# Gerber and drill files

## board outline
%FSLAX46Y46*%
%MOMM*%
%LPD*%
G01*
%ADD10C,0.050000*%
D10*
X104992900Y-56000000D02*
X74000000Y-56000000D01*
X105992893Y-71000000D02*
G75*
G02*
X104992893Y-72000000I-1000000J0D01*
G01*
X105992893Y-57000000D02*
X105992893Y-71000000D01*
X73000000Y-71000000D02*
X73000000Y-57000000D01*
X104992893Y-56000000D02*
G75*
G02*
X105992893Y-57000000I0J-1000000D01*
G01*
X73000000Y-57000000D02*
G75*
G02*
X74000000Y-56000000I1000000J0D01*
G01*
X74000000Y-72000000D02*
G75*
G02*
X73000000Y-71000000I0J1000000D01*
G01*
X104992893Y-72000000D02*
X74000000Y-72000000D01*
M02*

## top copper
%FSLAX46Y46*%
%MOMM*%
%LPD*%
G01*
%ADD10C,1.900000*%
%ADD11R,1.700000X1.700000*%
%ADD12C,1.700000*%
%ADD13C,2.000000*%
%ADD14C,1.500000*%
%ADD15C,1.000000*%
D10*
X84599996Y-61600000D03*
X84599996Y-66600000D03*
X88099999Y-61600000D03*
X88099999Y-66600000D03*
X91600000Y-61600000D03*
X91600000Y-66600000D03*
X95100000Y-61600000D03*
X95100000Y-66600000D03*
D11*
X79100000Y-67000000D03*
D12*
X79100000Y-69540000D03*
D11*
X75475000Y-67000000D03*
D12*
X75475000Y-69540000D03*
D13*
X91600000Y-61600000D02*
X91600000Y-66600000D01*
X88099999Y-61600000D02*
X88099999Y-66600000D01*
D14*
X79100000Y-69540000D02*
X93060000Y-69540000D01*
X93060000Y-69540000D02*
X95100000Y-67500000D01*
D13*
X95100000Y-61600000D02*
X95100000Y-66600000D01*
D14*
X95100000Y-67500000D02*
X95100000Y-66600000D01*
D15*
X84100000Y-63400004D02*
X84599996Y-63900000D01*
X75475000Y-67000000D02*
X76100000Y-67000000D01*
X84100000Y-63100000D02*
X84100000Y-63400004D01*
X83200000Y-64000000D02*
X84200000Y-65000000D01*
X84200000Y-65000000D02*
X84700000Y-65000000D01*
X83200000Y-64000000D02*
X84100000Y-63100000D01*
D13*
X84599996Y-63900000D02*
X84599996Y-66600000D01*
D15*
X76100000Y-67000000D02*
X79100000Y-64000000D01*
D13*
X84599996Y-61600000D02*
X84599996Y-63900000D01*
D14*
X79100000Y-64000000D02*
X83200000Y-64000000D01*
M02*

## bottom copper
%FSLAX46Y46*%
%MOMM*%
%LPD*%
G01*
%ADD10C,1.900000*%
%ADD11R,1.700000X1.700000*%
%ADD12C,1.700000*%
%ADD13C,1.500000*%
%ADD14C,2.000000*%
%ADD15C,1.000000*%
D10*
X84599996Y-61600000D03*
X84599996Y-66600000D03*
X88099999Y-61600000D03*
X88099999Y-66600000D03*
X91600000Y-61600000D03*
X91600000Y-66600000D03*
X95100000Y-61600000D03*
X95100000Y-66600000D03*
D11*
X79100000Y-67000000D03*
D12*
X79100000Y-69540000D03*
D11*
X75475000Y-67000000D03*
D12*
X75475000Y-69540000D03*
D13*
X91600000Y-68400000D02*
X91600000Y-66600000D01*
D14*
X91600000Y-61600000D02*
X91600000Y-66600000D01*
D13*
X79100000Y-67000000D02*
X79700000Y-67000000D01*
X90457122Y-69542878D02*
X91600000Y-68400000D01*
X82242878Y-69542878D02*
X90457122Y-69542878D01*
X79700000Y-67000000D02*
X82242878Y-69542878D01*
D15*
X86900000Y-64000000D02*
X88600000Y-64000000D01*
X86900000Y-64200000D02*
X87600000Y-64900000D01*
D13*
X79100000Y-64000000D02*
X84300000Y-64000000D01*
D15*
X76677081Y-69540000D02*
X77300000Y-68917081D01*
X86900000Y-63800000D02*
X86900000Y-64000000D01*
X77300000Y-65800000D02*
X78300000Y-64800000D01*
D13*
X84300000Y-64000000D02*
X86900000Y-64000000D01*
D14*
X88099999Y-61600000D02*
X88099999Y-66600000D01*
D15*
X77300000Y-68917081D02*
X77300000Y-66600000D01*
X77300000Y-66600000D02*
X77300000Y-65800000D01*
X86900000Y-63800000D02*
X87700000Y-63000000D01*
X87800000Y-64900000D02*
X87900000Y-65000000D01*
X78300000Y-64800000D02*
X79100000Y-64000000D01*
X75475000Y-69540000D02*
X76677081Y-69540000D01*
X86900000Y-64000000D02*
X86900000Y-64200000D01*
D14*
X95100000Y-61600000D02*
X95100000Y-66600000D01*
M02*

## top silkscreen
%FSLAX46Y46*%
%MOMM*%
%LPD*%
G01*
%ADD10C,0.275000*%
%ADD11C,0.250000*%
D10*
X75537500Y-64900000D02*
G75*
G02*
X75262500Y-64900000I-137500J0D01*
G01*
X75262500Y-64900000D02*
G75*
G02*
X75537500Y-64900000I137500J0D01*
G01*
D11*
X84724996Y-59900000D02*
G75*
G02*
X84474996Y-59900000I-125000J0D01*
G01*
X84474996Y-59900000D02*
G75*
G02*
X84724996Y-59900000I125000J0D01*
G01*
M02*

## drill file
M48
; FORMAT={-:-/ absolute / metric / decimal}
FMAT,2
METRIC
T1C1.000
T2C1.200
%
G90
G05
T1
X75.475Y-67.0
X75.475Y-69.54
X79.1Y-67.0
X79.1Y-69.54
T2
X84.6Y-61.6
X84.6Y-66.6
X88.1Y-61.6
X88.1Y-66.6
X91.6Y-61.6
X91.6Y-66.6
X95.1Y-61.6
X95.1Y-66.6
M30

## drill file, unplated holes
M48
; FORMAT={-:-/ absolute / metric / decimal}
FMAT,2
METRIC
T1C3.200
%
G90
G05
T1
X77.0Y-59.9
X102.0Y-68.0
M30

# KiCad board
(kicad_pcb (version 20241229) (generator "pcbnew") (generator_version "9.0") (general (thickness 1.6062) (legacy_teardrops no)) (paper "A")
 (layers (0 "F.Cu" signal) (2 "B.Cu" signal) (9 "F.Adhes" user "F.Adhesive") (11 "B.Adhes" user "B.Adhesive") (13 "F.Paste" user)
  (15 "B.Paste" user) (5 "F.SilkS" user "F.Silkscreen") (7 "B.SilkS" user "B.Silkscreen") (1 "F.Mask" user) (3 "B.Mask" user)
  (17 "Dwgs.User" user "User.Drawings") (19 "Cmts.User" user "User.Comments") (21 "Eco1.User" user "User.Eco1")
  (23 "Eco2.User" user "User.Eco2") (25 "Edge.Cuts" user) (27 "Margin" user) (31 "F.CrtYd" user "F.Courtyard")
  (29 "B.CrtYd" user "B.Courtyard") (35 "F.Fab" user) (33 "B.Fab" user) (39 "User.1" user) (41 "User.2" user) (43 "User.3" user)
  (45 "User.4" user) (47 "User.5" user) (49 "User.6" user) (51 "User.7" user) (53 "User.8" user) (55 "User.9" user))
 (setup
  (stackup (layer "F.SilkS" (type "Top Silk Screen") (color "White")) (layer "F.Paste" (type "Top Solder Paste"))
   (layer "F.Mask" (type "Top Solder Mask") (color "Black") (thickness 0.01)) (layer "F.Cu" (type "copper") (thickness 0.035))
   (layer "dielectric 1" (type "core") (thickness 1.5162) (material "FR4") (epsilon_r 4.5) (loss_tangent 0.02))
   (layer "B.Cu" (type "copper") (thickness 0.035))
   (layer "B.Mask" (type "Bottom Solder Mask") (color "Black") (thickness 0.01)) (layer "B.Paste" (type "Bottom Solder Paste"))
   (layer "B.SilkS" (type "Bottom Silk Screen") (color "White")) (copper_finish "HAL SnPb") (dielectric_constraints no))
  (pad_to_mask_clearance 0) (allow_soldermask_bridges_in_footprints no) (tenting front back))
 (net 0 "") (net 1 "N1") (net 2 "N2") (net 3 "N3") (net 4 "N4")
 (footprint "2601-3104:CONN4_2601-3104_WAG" (layer "F.Cu") (at 84.599996 61.6)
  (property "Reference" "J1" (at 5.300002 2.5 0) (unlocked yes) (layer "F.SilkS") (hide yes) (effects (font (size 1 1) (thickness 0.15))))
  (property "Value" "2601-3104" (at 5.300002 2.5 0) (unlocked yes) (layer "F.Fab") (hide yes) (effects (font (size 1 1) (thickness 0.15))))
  (fp_circle (center 0 -1.7) (end 0.2 -1.7) (stroke (width 0.1) (type solid)) (fill yes) (layer "F.SilkS"))
  (pad "1" thru_hole circle (at 0 0) (size 1.9 1.9) (drill 1.2) (layers "*.Cu" "*.Mask") (remove_unused_layers no) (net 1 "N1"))
  (pad "1" thru_hole circle (at 0 5) (size 1.9 1.9) (drill 1.2) (layers "*.Cu" "*.Mask") (remove_unused_layers no) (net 1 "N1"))
  (pad "2" thru_hole circle (at 3.500003 0) (size 1.9 1.9) (drill 1.2) (layers "*.Cu" "*.Mask") (remove_unused_layers no) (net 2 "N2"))
  (pad "2" thru_hole circle (at 3.500003 5) (size 1.9 1.9) (drill 1.2) (layers "*.Cu" "*.Mask") (remove_unused_layers no) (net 2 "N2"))
  (pad "3" thru_hole circle (at 7.000004 0) (size 1.9 1.9) (drill 1.2) (layers "*.Cu" "*.Mask") (remove_unused_layers no) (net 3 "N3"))
  (pad "3" thru_hole circle (at 7.000004 5) (size 1.9 1.9) (drill 1.2) (layers "*.Cu" "*.Mask") (remove_unused_layers no) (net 3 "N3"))
  (pad "4" thru_hole circle (at 10.500004 0) (size 1.9 1.9) (drill 1.2) (layers "*.Cu" "*.Mask") (remove_unused_layers no) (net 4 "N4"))
  (pad "4" thru_hole circle (at 10.500004 5) (size 1.9 1.9) (drill 1.2) (layers "*.Cu" "*.Mask") (remove_unused_layers no) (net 4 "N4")))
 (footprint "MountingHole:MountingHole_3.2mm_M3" (layer "F.Cu") (at 102 68)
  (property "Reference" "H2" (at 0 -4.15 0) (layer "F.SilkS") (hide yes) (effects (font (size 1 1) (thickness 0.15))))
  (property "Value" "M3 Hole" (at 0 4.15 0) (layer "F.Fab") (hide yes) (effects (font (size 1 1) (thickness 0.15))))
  (pad "" np_thru_hole circle (at 0 0) (size 3.2 3.2) (drill 3.2) (layers "*.Cu" "*.Mask")))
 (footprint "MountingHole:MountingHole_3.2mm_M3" (layer "F.Cu") (at 77 59.9)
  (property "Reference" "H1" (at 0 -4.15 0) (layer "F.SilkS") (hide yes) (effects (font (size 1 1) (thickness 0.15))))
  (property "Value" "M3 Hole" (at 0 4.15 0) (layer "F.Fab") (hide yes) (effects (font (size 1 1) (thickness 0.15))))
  (pad "" np_thru_hole circle (at 0 0) (size 3.2 3.2) (drill 3.2) (layers "*.Cu" "*.Mask")))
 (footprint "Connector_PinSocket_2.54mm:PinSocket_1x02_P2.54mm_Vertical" (layer "B.Cu") (at 79.1 67 180)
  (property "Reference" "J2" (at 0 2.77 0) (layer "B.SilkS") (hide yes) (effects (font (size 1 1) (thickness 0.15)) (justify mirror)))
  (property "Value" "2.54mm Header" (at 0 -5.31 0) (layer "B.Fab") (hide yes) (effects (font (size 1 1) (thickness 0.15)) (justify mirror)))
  (pad "1" thru_hole rect (at 0 0 180) (size 1.7 1.7) (drill 1) (layers "*.Cu" "*.Mask") (remove_unused_layers no) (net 3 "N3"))
  (pad "2" thru_hole circle (at 0 -2.54 180) (size 1.7 1.7) (drill 1) (layers "*.Cu" "*.Mask") (remove_unused_layers no) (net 4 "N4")))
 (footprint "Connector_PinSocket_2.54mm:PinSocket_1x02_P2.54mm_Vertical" (layer "B.Cu") (at 75.475 67 180)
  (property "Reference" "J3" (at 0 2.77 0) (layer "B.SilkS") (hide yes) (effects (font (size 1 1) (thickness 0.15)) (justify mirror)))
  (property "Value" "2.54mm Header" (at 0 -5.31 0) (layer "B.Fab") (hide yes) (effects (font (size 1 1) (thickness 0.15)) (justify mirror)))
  (pad "1" thru_hole rect (at 0 0 180) (size 1.7 1.7) (drill 1) (layers "*.Cu" "*.Mask") (remove_unused_layers no) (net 1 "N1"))
  (pad "2" thru_hole circle (at 0 -2.54 180) (size 1.7 1.7) (drill 1) (layers "*.Cu" "*.Mask") (remove_unused_layers no) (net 2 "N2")))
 (gr_circle (center 75.4 64.9) (end 75.6 64.9) (stroke (width 0.15) (type solid)) (fill yes) (layer "F.SilkS"))
 (gr_line (start 104.9929 56) (end 74 56) (stroke (width 0.05) (type default)) (layer "Edge.Cuts"))
 (gr_arc (start 105.992893 71) (mid 105.7 71.707107) (end 104.992893 72) (stroke (width 0.05) (type default)) (layer "Edge.Cuts"))
 (gr_line (start 105.992893 57) (end 105.992893 71) (stroke (width 0.05) (type default)) (layer "Edge.Cuts"))
 (gr_line (start 73 71) (end 73 57) (stroke (width 0.05) (type default)) (layer "Edge.Cuts"))
 (gr_arc (start 104.992893 56) (mid 105.7 56.292893) (end 105.992893 57) (stroke (width 0.05) (type default)) (layer "Edge.Cuts"))
 (gr_arc (start 73 57) (mid 73.292893 56.292893) (end 74 56) (stroke (width 0.05) (type default)) (layer "Edge.Cuts"))
 (gr_arc (start 74 72) (mid 73.292893 71.707107) (end 73 71) (stroke (width 0.05) (type default)) (layer "Edge.Cuts"))
 (gr_line (start 104.992893 72) (end 74 72) (stroke (width 0.05) (type default)) (layer "Edge.Cuts"))
 (segment (start 91.6 61.6) (end 91.6 66.6) (width 2) (layer "F.Cu") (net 3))
 (segment (start 91.6 68.4) (end 91.6 66.6) (width 1.5) (layer "B.Cu") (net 3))
 (segment (start 91.6 61.6) (end 91.6 66.6) (width 2) (layer "B.Cu") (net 3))
 (segment (start 79.1 67) (end 79.7 67) (width 1.5) (layer "B.Cu") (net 3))
 (segment (start 90.457122 69.542878) (end 91.6 68.4) (width 1.5) (layer "B.Cu") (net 3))
 (segment (start 82.242878 69.542878) (end 90.457122 69.542878) (width 1.5) (layer "B.Cu") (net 3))
 (segment (start 79.7 67) (end 82.242878 69.542878) (width 1.5) (layer "B.Cu") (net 3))
 (segment (start 88.099999 61.6) (end 88.099999 66.6) (width 2) (layer "F.Cu") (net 2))
 (segment (start 86.9 64) (end 88.6 64) (width 1) (layer "B.Cu") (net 2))
 (segment (start 86.9 64.2) (end 87.6 64.9) (width 1) (layer "B.Cu") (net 2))
 (segment (start 79.1 64) (end 84.3 64) (width 1.5) (layer "B.Cu") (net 2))
 (segment (start 76.677081 69.54) (end 77.3 68.917081) (width 1) (layer "B.Cu") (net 2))
 (segment (start 86.9 63.8) (end 86.9 64) (width 1) (layer "B.Cu") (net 2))
 (segment (start 77.3 65.8) (end 78.3 64.8) (width 1) (layer "B.Cu") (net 2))
 (segment (start 84.3 64) (end 86.9 64) (width 1.5) (layer "B.Cu") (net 2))
 (segment (start 88.099999 61.6) (end 88.099999 66.6) (width 2) (layer "B.Cu") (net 2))
 (segment (start 77.3 68.917081) (end 77.3 66.6) (width 1) (layer "B.Cu") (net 2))
 (segment (start 77.3 66.6) (end 77.3 65.8) (width 1) (layer "B.Cu") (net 2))
 (segment (start 86.9 63.8) (end 87.7 63) (width 1) (layer "B.Cu") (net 2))
 (segment (start 87.8 64.9) (end 87.9 65) (width 1) (layer "B.Cu") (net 2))
 (segment (start 78.3 64.8) (end 79.1 64) (width 1) (layer "B.Cu") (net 2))
 (segment (start 75.475 69.54) (end 76.677081 69.54) (width 1) (layer "B.Cu") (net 2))
 (segment (start 86.9 64) (end 86.9 64.2) (width 1) (layer "B.Cu") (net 2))
 (segment (start 79.1 69.54) (end 93.06 69.54) (width 1.5) (layer "F.Cu") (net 4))
 (segment (start 93.06 69.54) (end 95.1 67.5) (width 1.5) (layer "F.Cu") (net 4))
 (segment (start 95.1 61.6) (end 95.1 66.6) (width 2) (layer "F.Cu") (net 4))
 (segment (start 95.1 67.5) (end 95.1 66.6) (width 1.5) (layer "F.Cu") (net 4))
 (segment (start 95.1 61.6) (end 95.1 66.6) (width 2) (layer "B.Cu") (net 4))
 (segment (start 84.1 63.400004) (end 84.599996 63.9) (width 1) (layer "F.Cu") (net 1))
 (segment (start 75.475 67) (end 76.1 67) (width 1) (layer "F.Cu") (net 1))
 (segment (start 84.1 63.1) (end 84.1 63.400004) (width 1) (layer "F.Cu") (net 1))
 (segment (start 83.2 64) (end 84.2 65) (width 1) (layer "F.Cu") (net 1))
 (segment (start 84.2 65) (end 84.7 65) (width 1) (layer "F.Cu") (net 1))
 (segment (start 83.2 64) (end 84.1 63.1) (width 1) (layer "F.Cu") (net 1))
 (segment (start 84.599996 63.9) (end 84.599996 66.6) (width 2) (layer "F.Cu") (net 1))
 (segment (start 76.1 67) (end 79.1 64) (width 1) (layer "F.Cu") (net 1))
 (segment (start 84.599996 61.6) (end 84.599996 63.9) (width 2) (layer "F.Cu") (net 1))
 (segment (start 79.1 64) (end 83.2 64) (width 1.5) (layer "F.Cu") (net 1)))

